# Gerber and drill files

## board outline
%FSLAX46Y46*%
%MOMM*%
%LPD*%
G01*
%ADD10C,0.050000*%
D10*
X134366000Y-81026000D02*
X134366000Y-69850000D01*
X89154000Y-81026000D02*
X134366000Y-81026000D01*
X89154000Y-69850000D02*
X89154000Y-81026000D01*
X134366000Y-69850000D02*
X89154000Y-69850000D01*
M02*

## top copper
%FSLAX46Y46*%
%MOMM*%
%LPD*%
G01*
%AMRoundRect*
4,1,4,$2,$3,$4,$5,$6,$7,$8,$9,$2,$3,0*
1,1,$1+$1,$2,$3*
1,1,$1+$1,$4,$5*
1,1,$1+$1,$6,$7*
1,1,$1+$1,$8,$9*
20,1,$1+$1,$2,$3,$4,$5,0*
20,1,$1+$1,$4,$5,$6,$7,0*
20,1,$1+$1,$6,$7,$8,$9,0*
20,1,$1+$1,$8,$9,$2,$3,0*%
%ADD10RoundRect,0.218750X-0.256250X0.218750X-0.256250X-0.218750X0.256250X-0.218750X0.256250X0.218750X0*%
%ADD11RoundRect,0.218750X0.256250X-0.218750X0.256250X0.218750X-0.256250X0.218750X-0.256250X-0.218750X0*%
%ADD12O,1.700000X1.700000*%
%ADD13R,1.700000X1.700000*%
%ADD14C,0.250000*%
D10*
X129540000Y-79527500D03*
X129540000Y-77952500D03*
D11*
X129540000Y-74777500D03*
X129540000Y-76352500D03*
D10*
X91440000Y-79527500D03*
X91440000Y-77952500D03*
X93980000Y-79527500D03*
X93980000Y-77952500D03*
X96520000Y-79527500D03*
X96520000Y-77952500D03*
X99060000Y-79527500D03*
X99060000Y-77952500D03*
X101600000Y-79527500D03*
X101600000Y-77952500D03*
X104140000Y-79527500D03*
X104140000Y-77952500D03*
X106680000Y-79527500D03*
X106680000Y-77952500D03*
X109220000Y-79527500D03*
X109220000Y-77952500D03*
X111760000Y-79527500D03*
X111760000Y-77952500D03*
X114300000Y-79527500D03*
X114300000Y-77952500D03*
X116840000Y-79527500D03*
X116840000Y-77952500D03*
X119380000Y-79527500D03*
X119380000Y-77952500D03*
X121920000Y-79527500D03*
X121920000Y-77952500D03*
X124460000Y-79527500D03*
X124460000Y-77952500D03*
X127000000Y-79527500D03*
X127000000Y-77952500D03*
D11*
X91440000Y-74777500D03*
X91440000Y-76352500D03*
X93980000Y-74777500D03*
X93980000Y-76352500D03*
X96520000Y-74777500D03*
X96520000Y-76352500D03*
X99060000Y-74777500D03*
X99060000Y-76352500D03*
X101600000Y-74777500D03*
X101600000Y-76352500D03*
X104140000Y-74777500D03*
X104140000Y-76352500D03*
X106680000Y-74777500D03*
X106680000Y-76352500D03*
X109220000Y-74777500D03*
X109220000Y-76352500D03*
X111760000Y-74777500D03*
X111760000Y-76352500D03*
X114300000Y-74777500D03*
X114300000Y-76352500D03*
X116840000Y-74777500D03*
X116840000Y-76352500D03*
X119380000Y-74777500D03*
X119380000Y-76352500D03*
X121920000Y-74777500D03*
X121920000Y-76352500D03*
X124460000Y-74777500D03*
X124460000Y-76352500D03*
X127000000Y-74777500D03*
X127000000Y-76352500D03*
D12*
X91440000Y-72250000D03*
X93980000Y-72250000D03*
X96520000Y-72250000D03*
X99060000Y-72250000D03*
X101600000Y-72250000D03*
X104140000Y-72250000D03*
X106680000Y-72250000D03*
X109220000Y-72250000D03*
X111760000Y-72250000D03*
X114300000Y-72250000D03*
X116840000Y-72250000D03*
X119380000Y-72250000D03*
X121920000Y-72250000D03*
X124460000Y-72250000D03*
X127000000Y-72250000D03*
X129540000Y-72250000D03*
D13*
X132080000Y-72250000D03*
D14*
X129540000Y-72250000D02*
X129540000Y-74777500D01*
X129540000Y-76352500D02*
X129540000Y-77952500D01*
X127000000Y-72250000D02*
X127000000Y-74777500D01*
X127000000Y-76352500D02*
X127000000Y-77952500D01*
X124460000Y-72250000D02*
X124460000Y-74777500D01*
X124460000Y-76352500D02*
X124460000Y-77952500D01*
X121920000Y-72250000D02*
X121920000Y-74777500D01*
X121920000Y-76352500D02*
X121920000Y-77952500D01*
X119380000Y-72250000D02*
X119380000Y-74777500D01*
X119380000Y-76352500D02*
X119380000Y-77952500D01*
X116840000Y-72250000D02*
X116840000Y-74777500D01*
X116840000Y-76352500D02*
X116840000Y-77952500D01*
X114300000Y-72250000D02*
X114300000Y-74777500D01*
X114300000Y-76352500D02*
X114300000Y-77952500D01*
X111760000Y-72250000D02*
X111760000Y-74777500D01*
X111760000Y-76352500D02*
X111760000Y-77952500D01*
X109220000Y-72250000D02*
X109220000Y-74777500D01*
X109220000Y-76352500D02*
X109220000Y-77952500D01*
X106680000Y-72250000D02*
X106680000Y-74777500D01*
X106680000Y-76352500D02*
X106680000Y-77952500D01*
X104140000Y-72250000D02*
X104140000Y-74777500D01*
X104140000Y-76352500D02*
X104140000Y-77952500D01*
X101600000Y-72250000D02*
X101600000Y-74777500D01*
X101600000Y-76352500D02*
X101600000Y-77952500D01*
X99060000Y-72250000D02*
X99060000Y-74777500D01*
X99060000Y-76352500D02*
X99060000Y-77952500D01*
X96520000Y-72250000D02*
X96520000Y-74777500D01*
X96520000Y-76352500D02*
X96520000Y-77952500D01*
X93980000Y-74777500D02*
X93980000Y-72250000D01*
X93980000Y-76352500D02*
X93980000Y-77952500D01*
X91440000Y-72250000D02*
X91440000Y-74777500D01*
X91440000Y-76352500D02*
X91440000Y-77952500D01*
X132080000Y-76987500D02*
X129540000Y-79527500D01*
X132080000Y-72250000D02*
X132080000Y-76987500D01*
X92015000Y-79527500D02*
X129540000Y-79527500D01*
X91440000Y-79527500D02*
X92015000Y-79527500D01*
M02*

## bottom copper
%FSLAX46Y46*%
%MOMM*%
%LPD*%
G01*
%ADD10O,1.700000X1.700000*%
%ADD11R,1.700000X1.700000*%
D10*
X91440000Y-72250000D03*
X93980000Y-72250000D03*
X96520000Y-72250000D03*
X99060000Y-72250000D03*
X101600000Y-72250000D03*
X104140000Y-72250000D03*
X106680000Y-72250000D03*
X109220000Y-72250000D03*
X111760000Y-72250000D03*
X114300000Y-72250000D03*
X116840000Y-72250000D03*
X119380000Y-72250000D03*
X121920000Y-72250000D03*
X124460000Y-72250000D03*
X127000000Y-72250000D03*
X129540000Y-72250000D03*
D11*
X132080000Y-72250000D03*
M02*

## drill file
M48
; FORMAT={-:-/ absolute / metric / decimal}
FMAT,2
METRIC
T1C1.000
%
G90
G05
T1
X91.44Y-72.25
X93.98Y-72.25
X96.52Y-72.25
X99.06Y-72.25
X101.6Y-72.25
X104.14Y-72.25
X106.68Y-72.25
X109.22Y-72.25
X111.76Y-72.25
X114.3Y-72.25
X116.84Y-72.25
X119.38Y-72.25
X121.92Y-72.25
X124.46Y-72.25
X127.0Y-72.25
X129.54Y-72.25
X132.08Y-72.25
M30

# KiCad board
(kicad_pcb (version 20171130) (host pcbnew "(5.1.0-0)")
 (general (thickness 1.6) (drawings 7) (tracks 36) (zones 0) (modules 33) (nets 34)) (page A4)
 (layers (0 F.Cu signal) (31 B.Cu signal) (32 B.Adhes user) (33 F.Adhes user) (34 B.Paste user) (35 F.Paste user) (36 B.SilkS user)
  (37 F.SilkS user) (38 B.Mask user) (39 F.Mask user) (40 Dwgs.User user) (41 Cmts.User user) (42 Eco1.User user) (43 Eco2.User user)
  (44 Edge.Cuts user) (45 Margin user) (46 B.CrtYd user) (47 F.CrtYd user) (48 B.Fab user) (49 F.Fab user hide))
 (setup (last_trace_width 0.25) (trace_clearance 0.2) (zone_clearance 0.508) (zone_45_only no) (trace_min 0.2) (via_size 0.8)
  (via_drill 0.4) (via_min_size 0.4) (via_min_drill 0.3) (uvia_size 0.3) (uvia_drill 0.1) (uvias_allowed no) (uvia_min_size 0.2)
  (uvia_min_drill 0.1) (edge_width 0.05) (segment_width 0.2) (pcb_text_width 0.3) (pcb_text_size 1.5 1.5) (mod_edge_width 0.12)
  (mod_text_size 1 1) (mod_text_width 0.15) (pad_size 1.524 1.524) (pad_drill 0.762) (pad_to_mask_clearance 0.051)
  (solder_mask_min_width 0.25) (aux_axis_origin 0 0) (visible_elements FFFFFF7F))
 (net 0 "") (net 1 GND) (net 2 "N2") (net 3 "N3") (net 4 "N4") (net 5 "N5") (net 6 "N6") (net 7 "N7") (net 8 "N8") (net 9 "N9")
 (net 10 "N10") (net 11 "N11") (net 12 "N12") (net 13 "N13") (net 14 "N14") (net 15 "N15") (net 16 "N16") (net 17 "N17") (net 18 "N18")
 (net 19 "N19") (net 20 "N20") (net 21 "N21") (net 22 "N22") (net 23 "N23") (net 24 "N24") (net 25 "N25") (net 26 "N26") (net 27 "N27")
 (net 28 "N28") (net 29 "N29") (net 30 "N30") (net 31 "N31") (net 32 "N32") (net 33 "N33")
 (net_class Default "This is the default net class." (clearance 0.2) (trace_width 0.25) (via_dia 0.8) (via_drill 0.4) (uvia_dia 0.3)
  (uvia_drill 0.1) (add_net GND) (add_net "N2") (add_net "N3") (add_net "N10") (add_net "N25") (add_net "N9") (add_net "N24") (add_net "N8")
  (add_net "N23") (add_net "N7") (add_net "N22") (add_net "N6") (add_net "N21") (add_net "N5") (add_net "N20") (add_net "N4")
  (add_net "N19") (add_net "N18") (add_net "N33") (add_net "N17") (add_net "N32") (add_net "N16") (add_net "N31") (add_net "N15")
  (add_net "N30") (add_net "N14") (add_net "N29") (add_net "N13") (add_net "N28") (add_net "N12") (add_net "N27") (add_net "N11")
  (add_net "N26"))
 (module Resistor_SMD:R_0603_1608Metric (layer F.Cu) (at 129.54 78.74 270)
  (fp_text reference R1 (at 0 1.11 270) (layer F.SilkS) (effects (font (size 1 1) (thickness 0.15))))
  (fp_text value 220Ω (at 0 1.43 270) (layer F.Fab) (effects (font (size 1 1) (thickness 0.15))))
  (pad 2 smd roundrect (at 0.7875 0 270) (size 0.875 0.95) (layers F.Cu F.Paste F.Mask) (roundrect_rratio 0.25) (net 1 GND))
  (pad 1 smd roundrect (at -0.7875 0 270) (size 0.875 0.95) (layers F.Cu F.Paste F.Mask) (roundrect_rratio 0.25) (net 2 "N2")))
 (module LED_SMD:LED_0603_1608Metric (layer F.Cu) (at 129.54 75.565 90)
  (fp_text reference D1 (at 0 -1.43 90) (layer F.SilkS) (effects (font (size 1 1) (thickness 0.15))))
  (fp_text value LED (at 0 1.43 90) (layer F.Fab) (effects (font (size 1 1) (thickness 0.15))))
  (pad 2 smd roundrect (at 0.7875 0 90) (size 0.875 0.95) (layers F.Cu F.Paste F.Mask) (roundrect_rratio 0.25) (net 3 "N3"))
  (pad 1 smd roundrect (at -0.7875 0 90) (size 0.875 0.95) (layers F.Cu F.Paste F.Mask) (roundrect_rratio 0.25) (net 2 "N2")))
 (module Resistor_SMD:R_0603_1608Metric (layer F.Cu) (at 91.44 78.74 270)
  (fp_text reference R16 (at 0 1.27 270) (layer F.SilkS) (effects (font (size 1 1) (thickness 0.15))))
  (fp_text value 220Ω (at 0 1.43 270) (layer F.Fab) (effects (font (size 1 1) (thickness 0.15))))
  (pad 2 smd roundrect (at 0.7875 0 270) (size 0.875 0.95) (layers F.Cu F.Paste F.Mask) (roundrect_rratio 0.25) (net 1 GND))
  (pad 1 smd roundrect (at -0.7875 0 270) (size 0.875 0.95) (layers F.Cu F.Paste F.Mask) (roundrect_rratio 0.25) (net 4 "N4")))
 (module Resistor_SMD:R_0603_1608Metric (layer F.Cu) (at 93.98 78.74 270)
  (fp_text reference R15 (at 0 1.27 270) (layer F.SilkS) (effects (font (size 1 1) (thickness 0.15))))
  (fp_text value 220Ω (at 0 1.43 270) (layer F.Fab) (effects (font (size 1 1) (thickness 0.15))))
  (pad 2 smd roundrect (at 0.7875 0 270) (size 0.875 0.95) (layers F.Cu F.Paste F.Mask) (roundrect_rratio 0.25) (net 1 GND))
  (pad 1 smd roundrect (at -0.7875 0 270) (size 0.875 0.95) (layers F.Cu F.Paste F.Mask) (roundrect_rratio 0.25) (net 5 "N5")))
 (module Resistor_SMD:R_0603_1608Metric (layer F.Cu) (at 96.52 78.74 270)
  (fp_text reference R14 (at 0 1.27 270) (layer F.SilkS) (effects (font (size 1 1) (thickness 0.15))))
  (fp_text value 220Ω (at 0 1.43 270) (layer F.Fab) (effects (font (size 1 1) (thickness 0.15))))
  (pad 2 smd roundrect (at 0.7875 0 270) (size 0.875 0.95) (layers F.Cu F.Paste F.Mask) (roundrect_rratio 0.25) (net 1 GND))
  (pad 1 smd roundrect (at -0.7875 0 270) (size 0.875 0.95) (layers F.Cu F.Paste F.Mask) (roundrect_rratio 0.25) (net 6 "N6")))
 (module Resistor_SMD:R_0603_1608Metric (layer F.Cu) (at 99.06 78.74 270)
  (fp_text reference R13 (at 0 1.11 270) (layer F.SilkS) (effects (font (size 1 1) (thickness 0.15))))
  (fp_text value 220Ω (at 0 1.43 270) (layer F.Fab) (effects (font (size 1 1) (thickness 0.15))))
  (pad 2 smd roundrect (at 0.7875 0 270) (size 0.875 0.95) (layers F.Cu F.Paste F.Mask) (roundrect_rratio 0.25) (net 1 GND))
  (pad 1 smd roundrect (at -0.7875 0 270) (size 0.875 0.95) (layers F.Cu F.Paste F.Mask) (roundrect_rratio 0.25) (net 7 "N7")))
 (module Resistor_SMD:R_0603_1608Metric (layer F.Cu) (at 101.6 78.74 270)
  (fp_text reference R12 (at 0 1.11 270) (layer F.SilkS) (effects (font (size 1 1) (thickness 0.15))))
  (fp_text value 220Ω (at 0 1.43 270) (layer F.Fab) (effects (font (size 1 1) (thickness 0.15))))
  (pad 2 smd roundrect (at 0.7875 0 270) (size 0.875 0.95) (layers F.Cu F.Paste F.Mask) (roundrect_rratio 0.25) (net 1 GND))
  (pad 1 smd roundrect (at -0.7875 0 270) (size 0.875 0.95) (layers F.Cu F.Paste F.Mask) (roundrect_rratio 0.25) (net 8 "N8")))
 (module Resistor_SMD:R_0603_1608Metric (layer F.Cu) (at 104.14 78.74 270)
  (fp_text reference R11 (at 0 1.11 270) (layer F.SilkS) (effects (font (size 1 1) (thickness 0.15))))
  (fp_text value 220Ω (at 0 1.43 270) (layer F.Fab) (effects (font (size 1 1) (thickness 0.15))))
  (pad 2 smd roundrect (at 0.7875 0 270) (size 0.875 0.95) (layers F.Cu F.Paste F.Mask) (roundrect_rratio 0.25) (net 1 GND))
  (pad 1 smd roundrect (at -0.7875 0 270) (size 0.875 0.95) (layers F.Cu F.Paste F.Mask) (roundrect_rratio 0.25) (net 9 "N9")))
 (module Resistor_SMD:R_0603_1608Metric (layer F.Cu) (at 106.68 78.74 270)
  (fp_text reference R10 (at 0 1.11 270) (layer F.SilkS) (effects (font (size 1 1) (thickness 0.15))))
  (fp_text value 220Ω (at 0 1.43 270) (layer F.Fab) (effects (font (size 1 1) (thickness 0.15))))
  (pad 2 smd roundrect (at 0.7875 0 270) (size 0.875 0.95) (layers F.Cu F.Paste F.Mask) (roundrect_rratio 0.25) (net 1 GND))
  (pad 1 smd roundrect (at -0.7875 0 270) (size 0.875 0.95) (layers F.Cu F.Paste F.Mask) (roundrect_rratio 0.25) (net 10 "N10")))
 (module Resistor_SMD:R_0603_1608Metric (layer F.Cu) (at 109.22 78.74 270)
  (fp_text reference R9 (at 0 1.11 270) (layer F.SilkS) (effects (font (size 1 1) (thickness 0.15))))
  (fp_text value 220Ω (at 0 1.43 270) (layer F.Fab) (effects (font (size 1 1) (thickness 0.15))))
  (pad 2 smd roundrect (at 0.7875 0 270) (size 0.875 0.95) (layers F.Cu F.Paste F.Mask) (roundrect_rratio 0.25) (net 1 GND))
  (pad 1 smd roundrect (at -0.7875 0 270) (size 0.875 0.95) (layers F.Cu F.Paste F.Mask) (roundrect_rratio 0.25) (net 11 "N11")))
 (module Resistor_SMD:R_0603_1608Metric (layer F.Cu) (at 111.76 78.74 270)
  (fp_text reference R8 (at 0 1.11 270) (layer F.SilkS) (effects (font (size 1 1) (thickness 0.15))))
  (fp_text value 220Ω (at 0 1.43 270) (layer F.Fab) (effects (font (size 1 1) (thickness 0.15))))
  (pad 2 smd roundrect (at 0.7875 0 270) (size 0.875 0.95) (layers F.Cu F.Paste F.Mask) (roundrect_rratio 0.25) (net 1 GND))
  (pad 1 smd roundrect (at -0.7875 0 270) (size 0.875 0.95) (layers F.Cu F.Paste F.Mask) (roundrect_rratio 0.25) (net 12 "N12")))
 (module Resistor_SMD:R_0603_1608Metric (layer F.Cu) (at 114.3 78.74 270)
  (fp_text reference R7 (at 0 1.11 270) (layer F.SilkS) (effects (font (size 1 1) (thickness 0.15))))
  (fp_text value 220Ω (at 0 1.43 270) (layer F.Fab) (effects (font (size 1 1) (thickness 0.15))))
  (pad 2 smd roundrect (at 0.7875 0 270) (size 0.875 0.95) (layers F.Cu F.Paste F.Mask) (roundrect_rratio 0.25) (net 1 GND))
  (pad 1 smd roundrect (at -0.7875 0 270) (size 0.875 0.95) (layers F.Cu F.Paste F.Mask) (roundrect_rratio 0.25) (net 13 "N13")))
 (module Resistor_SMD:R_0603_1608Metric (layer F.Cu) (at 116.84 78.74 270)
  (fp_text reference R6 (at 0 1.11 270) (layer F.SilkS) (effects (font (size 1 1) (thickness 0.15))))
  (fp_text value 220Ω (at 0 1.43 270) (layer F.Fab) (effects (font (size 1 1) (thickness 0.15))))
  (pad 2 smd roundrect (at 0.7875 0 270) (size 0.875 0.95) (layers F.Cu F.Paste F.Mask) (roundrect_rratio 0.25) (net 1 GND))
  (pad 1 smd roundrect (at -0.7875 0 270) (size 0.875 0.95) (layers F.Cu F.Paste F.Mask) (roundrect_rratio 0.25) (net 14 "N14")))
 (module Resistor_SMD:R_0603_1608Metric (layer F.Cu) (at 119.38 78.74 270)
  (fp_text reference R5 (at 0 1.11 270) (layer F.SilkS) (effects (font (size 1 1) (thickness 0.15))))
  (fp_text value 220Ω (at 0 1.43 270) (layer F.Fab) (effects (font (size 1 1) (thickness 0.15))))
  (pad 2 smd roundrect (at 0.7875 0 270) (size 0.875 0.95) (layers F.Cu F.Paste F.Mask) (roundrect_rratio 0.25) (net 1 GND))
  (pad 1 smd roundrect (at -0.7875 0 270) (size 0.875 0.95) (layers F.Cu F.Paste F.Mask) (roundrect_rratio 0.25) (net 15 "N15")))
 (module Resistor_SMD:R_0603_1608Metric (layer F.Cu) (at 121.92 78.74 270)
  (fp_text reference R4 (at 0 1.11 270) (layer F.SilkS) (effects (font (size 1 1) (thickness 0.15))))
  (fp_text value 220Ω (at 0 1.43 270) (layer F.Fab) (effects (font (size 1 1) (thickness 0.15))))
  (pad 2 smd roundrect (at 0.7875 0 270) (size 0.875 0.95) (layers F.Cu F.Paste F.Mask) (roundrect_rratio 0.25) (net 1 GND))
  (pad 1 smd roundrect (at -0.7875 0 270) (size 0.875 0.95) (layers F.Cu F.Paste F.Mask) (roundrect_rratio 0.25) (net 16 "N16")))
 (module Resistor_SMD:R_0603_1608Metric (layer F.Cu) (at 124.46 78.74 270)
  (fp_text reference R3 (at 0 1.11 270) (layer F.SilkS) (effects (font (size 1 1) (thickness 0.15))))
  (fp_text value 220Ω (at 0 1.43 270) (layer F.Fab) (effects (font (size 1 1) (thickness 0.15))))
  (pad 2 smd roundrect (at 0.7875 0 270) (size 0.875 0.95) (layers F.Cu F.Paste F.Mask) (roundrect_rratio 0.25) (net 1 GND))
  (pad 1 smd roundrect (at -0.7875 0 270) (size 0.875 0.95) (layers F.Cu F.Paste F.Mask) (roundrect_rratio 0.25) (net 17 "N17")))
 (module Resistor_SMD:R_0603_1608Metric (layer F.Cu) (at 127 78.74 270)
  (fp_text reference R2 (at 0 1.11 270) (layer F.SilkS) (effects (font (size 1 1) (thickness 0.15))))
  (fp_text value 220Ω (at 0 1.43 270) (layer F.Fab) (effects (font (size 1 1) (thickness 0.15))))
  (pad 2 smd roundrect (at 0.7875 0 270) (size 0.875 0.95) (layers F.Cu F.Paste F.Mask) (roundrect_rratio 0.25) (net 1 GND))
  (pad 1 smd roundrect (at -0.7875 0 270) (size 0.875 0.95) (layers F.Cu F.Paste F.Mask) (roundrect_rratio 0.25) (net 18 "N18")))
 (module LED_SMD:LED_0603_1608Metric (layer F.Cu) (at 91.44 75.565 90)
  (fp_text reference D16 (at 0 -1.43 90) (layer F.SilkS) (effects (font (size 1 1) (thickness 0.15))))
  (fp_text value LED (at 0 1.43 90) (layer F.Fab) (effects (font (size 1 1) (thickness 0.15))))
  (pad 2 smd roundrect (at 0.7875 0 90) (size 0.875 0.95) (layers F.Cu F.Paste F.Mask) (roundrect_rratio 0.25) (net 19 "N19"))
  (pad 1 smd roundrect (at -0.7875 0 90) (size 0.875 0.95) (layers F.Cu F.Paste F.Mask) (roundrect_rratio 0.25) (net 4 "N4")))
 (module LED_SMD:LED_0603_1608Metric (layer F.Cu) (at 93.98 75.565 90)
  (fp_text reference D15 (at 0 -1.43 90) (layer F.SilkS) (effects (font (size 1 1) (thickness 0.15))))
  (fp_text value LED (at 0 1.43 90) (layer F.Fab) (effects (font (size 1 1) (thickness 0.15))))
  (pad 2 smd roundrect (at 0.7875 0 90) (size 0.875 0.95) (layers F.Cu F.Paste F.Mask) (roundrect_rratio 0.25) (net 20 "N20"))
  (pad 1 smd roundrect (at -0.7875 0 90) (size 0.875 0.95) (layers F.Cu F.Paste F.Mask) (roundrect_rratio 0.25) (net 5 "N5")))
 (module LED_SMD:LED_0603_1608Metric (layer F.Cu) (at 96.52 75.565 90)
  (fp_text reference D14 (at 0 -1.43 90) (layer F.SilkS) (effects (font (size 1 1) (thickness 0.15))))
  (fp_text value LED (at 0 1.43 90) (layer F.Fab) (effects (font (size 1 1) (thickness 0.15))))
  (pad 2 smd roundrect (at 0.7875 0 90) (size 0.875 0.95) (layers F.Cu F.Paste F.Mask) (roundrect_rratio 0.25) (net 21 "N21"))
  (pad 1 smd roundrect (at -0.7875 0 90) (size 0.875 0.95) (layers F.Cu F.Paste F.Mask) (roundrect_rratio 0.25) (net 6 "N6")))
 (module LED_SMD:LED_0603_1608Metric (layer F.Cu) (at 99.06 75.565 90)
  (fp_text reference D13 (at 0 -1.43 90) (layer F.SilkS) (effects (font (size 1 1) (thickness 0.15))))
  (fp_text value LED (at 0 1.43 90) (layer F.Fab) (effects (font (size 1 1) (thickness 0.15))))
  (pad 2 smd roundrect (at 0.7875 0 90) (size 0.875 0.95) (layers F.Cu F.Paste F.Mask) (roundrect_rratio 0.25) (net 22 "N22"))
  (pad 1 smd roundrect (at -0.7875 0 90) (size 0.875 0.95) (layers F.Cu F.Paste F.Mask) (roundrect_rratio 0.25) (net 7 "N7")))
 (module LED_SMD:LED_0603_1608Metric (layer F.Cu) (at 101.6 75.565 90)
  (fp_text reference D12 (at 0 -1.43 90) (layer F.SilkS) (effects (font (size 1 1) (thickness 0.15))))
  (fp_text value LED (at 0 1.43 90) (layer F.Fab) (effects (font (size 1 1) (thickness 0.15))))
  (pad 2 smd roundrect (at 0.7875 0 90) (size 0.875 0.95) (layers F.Cu F.Paste F.Mask) (roundrect_rratio 0.25) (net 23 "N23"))
  (pad 1 smd roundrect (at -0.7875 0 90) (size 0.875 0.95) (layers F.Cu F.Paste F.Mask) (roundrect_rratio 0.25) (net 8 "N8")))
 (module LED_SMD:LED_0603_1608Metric (layer F.Cu) (at 104.14 75.565 90)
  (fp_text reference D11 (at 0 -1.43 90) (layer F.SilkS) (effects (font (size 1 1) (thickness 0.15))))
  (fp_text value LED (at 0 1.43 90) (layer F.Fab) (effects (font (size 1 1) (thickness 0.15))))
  (pad 2 smd roundrect (at 0.7875 0 90) (size 0.875 0.95) (layers F.Cu F.Paste F.Mask) (roundrect_rratio 0.25) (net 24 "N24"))
  (pad 1 smd roundrect (at -0.7875 0 90) (size 0.875 0.95) (layers F.Cu F.Paste F.Mask) (roundrect_rratio 0.25) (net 9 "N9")))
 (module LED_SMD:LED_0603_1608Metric (layer F.Cu) (at 106.68 75.565 90)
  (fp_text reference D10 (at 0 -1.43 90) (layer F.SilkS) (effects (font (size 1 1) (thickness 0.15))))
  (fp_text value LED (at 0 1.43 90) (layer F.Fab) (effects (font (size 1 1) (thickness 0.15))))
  (pad 2 smd roundrect (at 0.7875 0 90) (size 0.875 0.95) (layers F.Cu F.Paste F.Mask) (roundrect_rratio 0.25) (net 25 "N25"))
  (pad 1 smd roundrect (at -0.7875 0 90) (size 0.875 0.95) (layers F.Cu F.Paste F.Mask) (roundrect_rratio 0.25) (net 10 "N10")))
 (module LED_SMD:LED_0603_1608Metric (layer F.Cu) (at 109.22 75.565 90)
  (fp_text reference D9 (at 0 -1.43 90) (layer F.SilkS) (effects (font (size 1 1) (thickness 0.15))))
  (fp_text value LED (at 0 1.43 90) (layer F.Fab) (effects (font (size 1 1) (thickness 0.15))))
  (pad 2 smd roundrect (at 0.7875 0 90) (size 0.875 0.95) (layers F.Cu F.Paste F.Mask) (roundrect_rratio 0.25) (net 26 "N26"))
  (pad 1 smd roundrect (at -0.7875 0 90) (size 0.875 0.95) (layers F.Cu F.Paste F.Mask) (roundrect_rratio 0.25) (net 11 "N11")))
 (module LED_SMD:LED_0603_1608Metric (layer F.Cu) (at 111.76 75.565 90)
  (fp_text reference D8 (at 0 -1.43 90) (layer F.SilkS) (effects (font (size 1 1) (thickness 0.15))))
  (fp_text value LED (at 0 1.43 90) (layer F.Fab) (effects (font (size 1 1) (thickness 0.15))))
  (pad 2 smd roundrect (at 0.7875 0 90) (size 0.875 0.95) (layers F.Cu F.Paste F.Mask) (roundrect_rratio 0.25) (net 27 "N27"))
  (pad 1 smd roundrect (at -0.7875 0 90) (size 0.875 0.95) (layers F.Cu F.Paste F.Mask) (roundrect_rratio 0.25) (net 12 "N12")))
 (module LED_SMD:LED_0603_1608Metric (layer F.Cu) (at 114.3 75.565 90)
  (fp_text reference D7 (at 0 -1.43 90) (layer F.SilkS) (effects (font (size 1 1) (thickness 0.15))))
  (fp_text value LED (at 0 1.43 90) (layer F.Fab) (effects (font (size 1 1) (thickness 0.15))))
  (pad 2 smd roundrect (at 0.7875 0 90) (size 0.875 0.95) (layers F.Cu F.Paste F.Mask) (roundrect_rratio 0.25) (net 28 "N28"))
  (pad 1 smd roundrect (at -0.7875 0 90) (size 0.875 0.95) (layers F.Cu F.Paste F.Mask) (roundrect_rratio 0.25) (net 13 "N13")))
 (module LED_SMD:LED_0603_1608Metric (layer F.Cu) (at 116.84 75.565 90)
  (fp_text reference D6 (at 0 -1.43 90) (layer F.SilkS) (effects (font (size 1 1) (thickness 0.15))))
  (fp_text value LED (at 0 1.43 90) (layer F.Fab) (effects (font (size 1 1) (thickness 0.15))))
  (pad 2 smd roundrect (at 0.7875 0 90) (size 0.875 0.95) (layers F.Cu F.Paste F.Mask) (roundrect_rratio 0.25) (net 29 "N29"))
  (pad 1 smd roundrect (at -0.7875 0 90) (size 0.875 0.95) (layers F.Cu F.Paste F.Mask) (roundrect_rratio 0.25) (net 14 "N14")))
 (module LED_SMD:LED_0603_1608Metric (layer F.Cu) (at 119.38 75.565 90)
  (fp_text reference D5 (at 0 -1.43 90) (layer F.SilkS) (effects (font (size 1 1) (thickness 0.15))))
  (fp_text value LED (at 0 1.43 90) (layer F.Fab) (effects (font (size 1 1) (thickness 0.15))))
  (pad 2 smd roundrect (at 0.7875 0 90) (size 0.875 0.95) (layers F.Cu F.Paste F.Mask) (roundrect_rratio 0.25) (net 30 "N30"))
  (pad 1 smd roundrect (at -0.7875 0 90) (size 0.875 0.95) (layers F.Cu F.Paste F.Mask) (roundrect_rratio 0.25) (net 15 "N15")))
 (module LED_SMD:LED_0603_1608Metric (layer F.Cu) (at 121.92 75.565 90)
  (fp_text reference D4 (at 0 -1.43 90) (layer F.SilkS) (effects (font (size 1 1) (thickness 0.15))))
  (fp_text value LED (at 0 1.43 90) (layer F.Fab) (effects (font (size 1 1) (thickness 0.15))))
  (pad 2 smd roundrect (at 0.7875 0 90) (size 0.875 0.95) (layers F.Cu F.Paste F.Mask) (roundrect_rratio 0.25) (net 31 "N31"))
  (pad 1 smd roundrect (at -0.7875 0 90) (size 0.875 0.95) (layers F.Cu F.Paste F.Mask) (roundrect_rratio 0.25) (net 16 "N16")))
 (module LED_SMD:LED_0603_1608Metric (layer F.Cu) (at 124.46 75.565 90)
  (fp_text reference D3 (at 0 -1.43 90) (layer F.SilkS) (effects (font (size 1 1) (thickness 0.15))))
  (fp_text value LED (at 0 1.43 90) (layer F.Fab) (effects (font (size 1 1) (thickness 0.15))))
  (pad 2 smd roundrect (at 0.7875 0 90) (size 0.875 0.95) (layers F.Cu F.Paste F.Mask) (roundrect_rratio 0.25) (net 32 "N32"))
  (pad 1 smd roundrect (at -0.7875 0 90) (size 0.875 0.95) (layers F.Cu F.Paste F.Mask) (roundrect_rratio 0.25) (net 17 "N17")))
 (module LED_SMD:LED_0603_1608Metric (layer F.Cu) (at 127 75.565 90)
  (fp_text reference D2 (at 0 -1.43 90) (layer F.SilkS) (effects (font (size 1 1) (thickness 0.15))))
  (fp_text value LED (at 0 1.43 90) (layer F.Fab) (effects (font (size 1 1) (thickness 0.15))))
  (pad 2 smd roundrect (at 0.7875 0 90) (size 0.875 0.95) (layers F.Cu F.Paste F.Mask) (roundrect_rratio 0.25) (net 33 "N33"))
  (pad 1 smd roundrect (at -0.7875 0 90) (size 0.875 0.95) (layers F.Cu F.Paste F.Mask) (roundrect_rratio 0.25) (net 18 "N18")))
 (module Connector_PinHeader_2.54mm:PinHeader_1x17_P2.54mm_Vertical (layer B.Cu) (at 132.08 72.25 90)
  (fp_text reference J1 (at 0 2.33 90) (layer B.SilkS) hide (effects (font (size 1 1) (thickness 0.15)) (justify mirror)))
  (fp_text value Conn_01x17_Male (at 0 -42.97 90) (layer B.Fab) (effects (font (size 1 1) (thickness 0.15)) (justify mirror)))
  (pad 17 thru_hole oval (at 0 -40.64 90) (size 1.7 1.7) (drill 1) (layers *.Cu *.Mask) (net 19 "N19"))
  (pad 16 thru_hole oval (at 0 -38.1 90) (size 1.7 1.7) (drill 1) (layers *.Cu *.Mask) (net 20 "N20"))
  (pad 15 thru_hole oval (at 0 -35.56 90) (size 1.7 1.7) (drill 1) (layers *.Cu *.Mask) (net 21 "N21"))
  (pad 14 thru_hole oval (at 0 -33.02 90) (size 1.7 1.7) (drill 1) (layers *.Cu *.Mask) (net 22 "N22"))
  (pad 13 thru_hole oval (at 0 -30.48 90) (size 1.7 1.7) (drill 1) (layers *.Cu *.Mask) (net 23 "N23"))
  (pad 12 thru_hole oval (at 0 -27.94 90) (size 1.7 1.7) (drill 1) (layers *.Cu *.Mask) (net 24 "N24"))
  (pad 11 thru_hole oval (at 0 -25.4 90) (size 1.7 1.7) (drill 1) (layers *.Cu *.Mask) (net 25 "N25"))
  (pad 10 thru_hole oval (at 0 -22.86 90) (size 1.7 1.7) (drill 1) (layers *.Cu *.Mask) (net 26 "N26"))
  (pad 9 thru_hole oval (at 0 -20.32 90) (size 1.7 1.7) (drill 1) (layers *.Cu *.Mask) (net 27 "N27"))
  (pad 8 thru_hole oval (at 0 -17.78 90) (size 1.7 1.7) (drill 1) (layers *.Cu *.Mask) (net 28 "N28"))
  (pad 7 thru_hole oval (at 0 -15.24 90) (size 1.7 1.7) (drill 1) (layers *.Cu *.Mask) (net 29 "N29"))
  (pad 6 thru_hole oval (at 0 -12.7 90) (size 1.7 1.7) (drill 1) (layers *.Cu *.Mask) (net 30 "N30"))
  (pad 5 thru_hole oval (at 0 -10.16 90) (size 1.7 1.7) (drill 1) (layers *.Cu *.Mask) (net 31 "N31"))
  (pad 4 thru_hole oval (at 0 -7.62 90) (size 1.7 1.7) (drill 1) (layers *.Cu *.Mask) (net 32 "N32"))
  (pad 3 thru_hole oval (at 0 -5.08 90) (size 1.7 1.7) (drill 1) (layers *.Cu *.Mask) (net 33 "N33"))
  (pad 2 thru_hole oval (at 0 -2.54 90) (size 1.7 1.7) (drill 1) (layers *.Cu *.Mask) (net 3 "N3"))
  (pad 1 thru_hole rect (at 0 0 90) (size 1.7 1.7) (drill 1) (layers *.Cu *.Mask) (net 1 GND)))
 (gr_line (start 134.366 81.026) (end 134.366 69.85) (layer Edge.Cuts) (width 0.05))
 (gr_line (start 89.154 81.026) (end 134.366 81.026) (layer Edge.Cuts) (width 0.05))
 (gr_line (start 89.154 69.85) (end 89.154 81.026) (layer Edge.Cuts) (width 0.05))
 (gr_line (start 134.366 69.85) (end 89.154 69.85) (layer Edge.Cuts) (width 0.05))
 (segment (start 129.54 72.25) (end 129.54 74.7775) (width 0.25) (layer F.Cu) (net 3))
 (segment (start 129.54 76.3525) (end 129.54 77.9525) (width 0.25) (layer F.Cu) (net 2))
 (segment (start 127 72.25) (end 127 74.7775) (width 0.25) (layer F.Cu) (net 33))
 (segment (start 127 76.3525) (end 127 77.9525) (width 0.25) (layer F.Cu) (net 18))
 (segment (start 124.46 72.25) (end 124.46 74.7775) (width 0.25) (layer F.Cu) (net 32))
 (segment (start 124.46 76.3525) (end 124.46 77.9525) (width 0.25) (layer F.Cu) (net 17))
 (segment (start 121.92 72.25) (end 121.92 74.7775) (width 0.25) (layer F.Cu) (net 31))
 (segment (start 121.92 76.3525) (end 121.92 77.9525) (width 0.25) (layer F.Cu) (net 16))
 (segment (start 119.38 72.25) (end 119.38 74.7775) (width 0.25) (layer F.Cu) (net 30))
 (segment (start 119.38 76.3525) (end 119.38 77.9525) (width 0.25) (layer F.Cu) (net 15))
 (segment (start 116.84 72.25) (end 116.84 74.7775) (width 0.25) (layer F.Cu) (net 29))
 (segment (start 116.84 76.3525) (end 116.84 77.9525) (width 0.25) (layer F.Cu) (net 14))
 (segment (start 114.3 72.25) (end 114.3 74.7775) (width 0.25) (layer F.Cu) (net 28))
 (segment (start 114.3 76.3525) (end 114.3 77.9525) (width 0.25) (layer F.Cu) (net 13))
 (segment (start 111.76 72.25) (end 111.76 74.7775) (width 0.25) (layer F.Cu) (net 27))
 (segment (start 111.76 76.3525) (end 111.76 77.9525) (width 0.25) (layer F.Cu) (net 12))
 (segment (start 109.22 72.25) (end 109.22 74.7775) (width 0.25) (layer F.Cu) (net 26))
 (segment (start 109.22 76.3525) (end 109.22 77.9525) (width 0.25) (layer F.Cu) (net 11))
 (segment (start 106.68 72.25) (end 106.68 74.7775) (width 0.25) (layer F.Cu) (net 25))
 (segment (start 106.68 76.3525) (end 106.68 77.9525) (width 0.25) (layer F.Cu) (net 10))
 (segment (start 104.14 72.25) (end 104.14 74.7775) (width 0.25) (layer F.Cu) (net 24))
 (segment (start 104.14 76.3525) (end 104.14 77.9525) (width 0.25) (layer F.Cu) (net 9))
 (segment (start 101.6 72.25) (end 101.6 74.7775) (width 0.25) (layer F.Cu) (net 23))
 (segment (start 101.6 76.3525) (end 101.6 77.9525) (width 0.25) (layer F.Cu) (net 8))
 (segment (start 99.06 72.25) (end 99.06 74.7775) (width 0.25) (layer F.Cu) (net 22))
 (segment (start 99.06 76.3525) (end 99.06 77.9525) (width 0.25) (layer F.Cu) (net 7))
 (segment (start 96.52 72.25) (end 96.52 74.7775) (width 0.25) (layer F.Cu) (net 21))
 (segment (start 96.52 76.3525) (end 96.52 77.9525) (width 0.25) (layer F.Cu) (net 6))
 (segment (start 93.98 74.7775) (end 93.98 72.25) (width 0.25) (layer F.Cu) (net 20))
 (segment (start 93.98 76.3525) (end 93.98 77.9525) (width 0.25) (layer F.Cu) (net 5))
 (segment (start 91.44 72.25) (end 91.44 74.7775) (width 0.25) (layer F.Cu) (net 19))
 (segment (start 91.44 76.3525) (end 91.44 77.9525) (width 0.25) (layer F.Cu) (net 4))
 (segment (start 132.08 76.9875) (end 129.54 79.5275) (width 0.25) (layer F.Cu) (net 1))
 (segment (start 132.08 72.25) (end 132.08 76.9875) (width 0.25) (layer F.Cu) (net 1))
 (segment (start 92.015 79.5275) (end 129.54 79.5275) (width 0.25) (layer F.Cu) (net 1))
 (segment (start 91.44 79.5275) (end 92.015 79.5275) (width 0.25) (layer F.Cu) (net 1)))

